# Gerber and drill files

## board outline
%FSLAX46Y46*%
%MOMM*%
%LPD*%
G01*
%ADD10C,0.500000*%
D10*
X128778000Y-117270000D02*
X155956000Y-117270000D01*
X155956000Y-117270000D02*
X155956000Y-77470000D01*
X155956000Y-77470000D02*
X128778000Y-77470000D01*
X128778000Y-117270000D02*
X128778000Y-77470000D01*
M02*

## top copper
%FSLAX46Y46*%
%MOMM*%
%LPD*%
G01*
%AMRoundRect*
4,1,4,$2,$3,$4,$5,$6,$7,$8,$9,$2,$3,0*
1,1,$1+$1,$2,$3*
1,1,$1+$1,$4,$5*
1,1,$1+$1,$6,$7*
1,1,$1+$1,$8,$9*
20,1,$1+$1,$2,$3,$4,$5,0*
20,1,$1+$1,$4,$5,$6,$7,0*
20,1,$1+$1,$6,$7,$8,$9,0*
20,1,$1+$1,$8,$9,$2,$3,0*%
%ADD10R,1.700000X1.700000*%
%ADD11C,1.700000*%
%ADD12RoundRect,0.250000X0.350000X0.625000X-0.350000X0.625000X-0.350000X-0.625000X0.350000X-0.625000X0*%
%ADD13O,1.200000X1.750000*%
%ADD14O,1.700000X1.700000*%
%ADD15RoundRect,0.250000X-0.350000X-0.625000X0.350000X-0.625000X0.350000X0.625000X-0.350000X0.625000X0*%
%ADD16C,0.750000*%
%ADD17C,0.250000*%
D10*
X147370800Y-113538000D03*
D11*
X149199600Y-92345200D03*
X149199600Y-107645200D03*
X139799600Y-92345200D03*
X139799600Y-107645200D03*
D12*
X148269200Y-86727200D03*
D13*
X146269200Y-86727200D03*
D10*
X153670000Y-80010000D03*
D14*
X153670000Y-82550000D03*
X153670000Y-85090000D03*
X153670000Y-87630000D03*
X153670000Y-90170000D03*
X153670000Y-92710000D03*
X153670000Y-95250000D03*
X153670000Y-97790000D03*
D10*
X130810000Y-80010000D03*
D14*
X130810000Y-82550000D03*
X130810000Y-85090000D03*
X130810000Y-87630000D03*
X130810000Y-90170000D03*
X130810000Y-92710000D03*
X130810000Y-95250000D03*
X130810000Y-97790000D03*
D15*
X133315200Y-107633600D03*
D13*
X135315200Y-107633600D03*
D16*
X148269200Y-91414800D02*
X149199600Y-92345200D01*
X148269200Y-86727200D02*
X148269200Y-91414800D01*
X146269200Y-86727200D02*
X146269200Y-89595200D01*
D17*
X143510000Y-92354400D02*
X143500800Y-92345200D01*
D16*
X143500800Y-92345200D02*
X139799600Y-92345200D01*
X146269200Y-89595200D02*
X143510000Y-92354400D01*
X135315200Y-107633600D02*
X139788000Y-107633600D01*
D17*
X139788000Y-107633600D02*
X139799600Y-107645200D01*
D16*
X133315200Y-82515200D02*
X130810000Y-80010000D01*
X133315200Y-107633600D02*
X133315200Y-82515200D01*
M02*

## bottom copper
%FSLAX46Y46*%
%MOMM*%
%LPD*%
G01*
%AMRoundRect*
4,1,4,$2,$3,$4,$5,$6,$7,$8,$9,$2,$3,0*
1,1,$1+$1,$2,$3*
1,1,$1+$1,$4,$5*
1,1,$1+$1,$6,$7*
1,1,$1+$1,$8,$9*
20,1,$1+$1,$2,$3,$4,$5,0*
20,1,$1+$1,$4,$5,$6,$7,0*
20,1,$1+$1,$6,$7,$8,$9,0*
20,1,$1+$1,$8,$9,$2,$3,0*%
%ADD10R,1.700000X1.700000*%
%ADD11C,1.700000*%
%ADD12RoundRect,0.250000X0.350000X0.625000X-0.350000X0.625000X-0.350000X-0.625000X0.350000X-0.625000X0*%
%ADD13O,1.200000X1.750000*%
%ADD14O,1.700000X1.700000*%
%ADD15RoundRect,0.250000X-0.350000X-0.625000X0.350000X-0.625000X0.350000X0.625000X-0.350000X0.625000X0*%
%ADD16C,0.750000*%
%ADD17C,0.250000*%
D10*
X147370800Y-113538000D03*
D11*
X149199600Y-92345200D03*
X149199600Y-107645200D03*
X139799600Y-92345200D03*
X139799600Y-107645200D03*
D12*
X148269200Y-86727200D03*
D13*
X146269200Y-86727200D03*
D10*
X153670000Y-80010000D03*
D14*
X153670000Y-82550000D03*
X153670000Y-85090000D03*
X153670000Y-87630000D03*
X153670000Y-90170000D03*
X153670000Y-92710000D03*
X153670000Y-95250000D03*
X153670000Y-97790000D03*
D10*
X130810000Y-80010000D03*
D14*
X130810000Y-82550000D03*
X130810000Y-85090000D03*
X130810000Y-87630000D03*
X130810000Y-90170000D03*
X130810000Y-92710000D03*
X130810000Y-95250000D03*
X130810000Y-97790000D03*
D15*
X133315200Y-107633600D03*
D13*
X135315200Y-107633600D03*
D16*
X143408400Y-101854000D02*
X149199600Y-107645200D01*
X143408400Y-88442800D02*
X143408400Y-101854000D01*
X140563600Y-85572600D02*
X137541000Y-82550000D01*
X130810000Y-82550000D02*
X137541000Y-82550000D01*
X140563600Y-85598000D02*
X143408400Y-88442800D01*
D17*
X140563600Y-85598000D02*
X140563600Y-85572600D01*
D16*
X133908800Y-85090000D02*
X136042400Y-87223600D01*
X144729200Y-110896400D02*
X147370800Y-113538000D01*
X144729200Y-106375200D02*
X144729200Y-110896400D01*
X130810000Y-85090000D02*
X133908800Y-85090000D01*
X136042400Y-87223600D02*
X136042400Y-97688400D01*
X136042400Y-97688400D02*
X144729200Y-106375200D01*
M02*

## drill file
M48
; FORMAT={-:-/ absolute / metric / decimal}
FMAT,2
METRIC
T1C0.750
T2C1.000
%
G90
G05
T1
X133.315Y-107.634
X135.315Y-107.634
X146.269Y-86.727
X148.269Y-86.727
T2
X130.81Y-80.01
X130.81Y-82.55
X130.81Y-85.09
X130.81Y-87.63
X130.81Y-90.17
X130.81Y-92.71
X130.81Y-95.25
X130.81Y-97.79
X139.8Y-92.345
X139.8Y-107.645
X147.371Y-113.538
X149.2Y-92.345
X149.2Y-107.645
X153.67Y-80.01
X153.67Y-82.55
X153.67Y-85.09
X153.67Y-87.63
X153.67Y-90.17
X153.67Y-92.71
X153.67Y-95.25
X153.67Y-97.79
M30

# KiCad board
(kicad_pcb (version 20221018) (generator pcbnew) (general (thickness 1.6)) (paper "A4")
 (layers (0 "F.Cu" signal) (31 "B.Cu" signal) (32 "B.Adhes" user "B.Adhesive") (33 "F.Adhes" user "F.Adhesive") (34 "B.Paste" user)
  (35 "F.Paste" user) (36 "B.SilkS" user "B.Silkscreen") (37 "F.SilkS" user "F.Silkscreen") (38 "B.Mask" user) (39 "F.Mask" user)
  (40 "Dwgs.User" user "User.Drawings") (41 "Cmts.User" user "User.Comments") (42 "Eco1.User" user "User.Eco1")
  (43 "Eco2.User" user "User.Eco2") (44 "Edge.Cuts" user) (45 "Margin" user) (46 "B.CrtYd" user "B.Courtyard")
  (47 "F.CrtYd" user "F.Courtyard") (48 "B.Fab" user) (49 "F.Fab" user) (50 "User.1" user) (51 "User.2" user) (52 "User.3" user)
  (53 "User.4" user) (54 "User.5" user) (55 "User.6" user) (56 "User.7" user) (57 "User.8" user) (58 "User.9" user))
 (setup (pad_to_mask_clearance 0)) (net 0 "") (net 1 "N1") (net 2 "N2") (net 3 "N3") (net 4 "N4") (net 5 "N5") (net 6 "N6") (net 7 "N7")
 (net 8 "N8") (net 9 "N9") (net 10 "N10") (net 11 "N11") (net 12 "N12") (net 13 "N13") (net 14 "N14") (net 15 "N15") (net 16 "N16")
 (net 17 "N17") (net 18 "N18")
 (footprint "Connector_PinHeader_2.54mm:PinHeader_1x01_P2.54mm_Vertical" (layer "F.Cu") (at 147.3708 113.538)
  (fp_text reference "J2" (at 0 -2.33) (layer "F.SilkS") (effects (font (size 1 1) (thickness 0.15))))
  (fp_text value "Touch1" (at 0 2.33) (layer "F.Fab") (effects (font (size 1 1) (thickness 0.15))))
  (pad "1" thru_hole rect (at 0 0) (size 1.7 1.7) (drill 1) (layers "*.Cu" "*.Mask") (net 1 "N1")))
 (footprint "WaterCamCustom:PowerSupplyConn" (layer "F.Cu") (at 144.4996 99.9952 -90)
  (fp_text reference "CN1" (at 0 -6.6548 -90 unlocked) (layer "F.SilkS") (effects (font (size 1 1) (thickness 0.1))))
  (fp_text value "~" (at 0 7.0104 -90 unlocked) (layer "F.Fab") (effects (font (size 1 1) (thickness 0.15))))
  (pad "1" thru_hole circle (at -7.65 -4.7 270) (size 1.7 1.7) (drill 1) (layers "*.Cu" "*.Mask") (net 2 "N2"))
  (pad "2" thru_hole circle (at 7.65 -4.7 270) (size 1.7 1.7) (drill 1) (layers "*.Cu" "*.Mask") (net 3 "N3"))
  (pad "3" thru_hole circle (at -7.65 4.7 270) (size 1.7 1.7) (drill 1) (layers "*.Cu" "*.Mask") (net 1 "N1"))
  (pad "4" thru_hole circle (at 7.65 4.7 270) (size 1.7 1.7) (drill 1) (layers "*.Cu" "*.Mask") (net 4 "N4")))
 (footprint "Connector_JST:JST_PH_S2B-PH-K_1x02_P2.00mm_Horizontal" (layer "F.Cu") (at 148.2692 86.7272 180)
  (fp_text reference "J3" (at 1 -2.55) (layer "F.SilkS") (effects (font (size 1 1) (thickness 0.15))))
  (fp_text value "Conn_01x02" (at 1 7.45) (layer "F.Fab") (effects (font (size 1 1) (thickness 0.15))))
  (pad "1" thru_hole roundrect (at 0 0 180) (size 1.2 1.75) (drill 0.75) (layers "*.Cu" "*.Mask") (roundrect_rratio 0.2083333333)
   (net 2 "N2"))
  (pad "2" thru_hole oval (at 2 0 180) (size 1.2 1.75) (drill 0.75) (layers "*.Cu" "*.Mask") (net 1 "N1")))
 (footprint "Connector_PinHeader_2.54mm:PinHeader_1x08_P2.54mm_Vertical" (layer "F.Cu") (at 153.67 80.01)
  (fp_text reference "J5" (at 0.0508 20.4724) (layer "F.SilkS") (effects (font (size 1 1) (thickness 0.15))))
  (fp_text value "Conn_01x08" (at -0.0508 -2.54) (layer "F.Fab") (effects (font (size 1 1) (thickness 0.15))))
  (pad "1" thru_hole rect (at 0 0) (size 1.7 1.7) (drill 1) (layers "*.Cu" "*.Mask") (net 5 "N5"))
  (pad "2" thru_hole oval (at 0 2.54) (size 1.7 1.7) (drill 1) (layers "*.Cu" "*.Mask") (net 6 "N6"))
  (pad "3" thru_hole oval (at 0 5.08) (size 1.7 1.7) (drill 1) (layers "*.Cu" "*.Mask") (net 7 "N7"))
  (pad "4" thru_hole oval (at 0 7.62) (size 1.7 1.7) (drill 1) (layers "*.Cu" "*.Mask") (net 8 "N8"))
  (pad "5" thru_hole oval (at 0 10.16) (size 1.7 1.7) (drill 1) (layers "*.Cu" "*.Mask") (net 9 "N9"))
  (pad "6" thru_hole oval (at 0 12.7) (size 1.7 1.7) (drill 1) (layers "*.Cu" "*.Mask") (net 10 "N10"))
  (pad "7" thru_hole oval (at 0 15.24) (size 1.7 1.7) (drill 1) (layers "*.Cu" "*.Mask") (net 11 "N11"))
  (pad "8" thru_hole oval (at 0 17.78) (size 1.7 1.7) (drill 1) (layers "*.Cu" "*.Mask") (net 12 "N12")))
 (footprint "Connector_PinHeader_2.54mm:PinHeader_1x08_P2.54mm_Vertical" (layer "F.Cu") (at 130.81 80.01)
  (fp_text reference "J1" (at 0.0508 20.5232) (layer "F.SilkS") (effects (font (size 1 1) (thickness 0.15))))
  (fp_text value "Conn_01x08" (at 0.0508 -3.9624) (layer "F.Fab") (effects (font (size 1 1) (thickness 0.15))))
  (pad "1" thru_hole rect (at 0 0) (size 1.7 1.7) (drill 1) (layers "*.Cu" "*.Mask") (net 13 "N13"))
  (pad "2" thru_hole oval (at 0 2.54) (size 1.7 1.7) (drill 1) (layers "*.Cu" "*.Mask") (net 3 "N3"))
  (pad "3" thru_hole oval (at 0 5.08) (size 1.7 1.7) (drill 1) (layers "*.Cu" "*.Mask") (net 1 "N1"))
  (pad "4" thru_hole oval (at 0 7.62) (size 1.7 1.7) (drill 1) (layers "*.Cu" "*.Mask") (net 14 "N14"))
  (pad "5" thru_hole oval (at 0 10.16) (size 1.7 1.7) (drill 1) (layers "*.Cu" "*.Mask") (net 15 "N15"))
  (pad "6" thru_hole oval (at 0 12.7) (size 1.7 1.7) (drill 1) (layers "*.Cu" "*.Mask") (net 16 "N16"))
  (pad "7" thru_hole oval (at 0 15.24) (size 1.7 1.7) (drill 1) (layers "*.Cu" "*.Mask") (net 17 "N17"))
  (pad "8" thru_hole oval (at 0 17.78) (size 1.7 1.7) (drill 1) (layers "*.Cu" "*.Mask") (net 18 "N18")))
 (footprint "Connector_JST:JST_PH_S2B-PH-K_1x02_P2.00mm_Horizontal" (layer "F.Cu") (at 133.3152 107.6336)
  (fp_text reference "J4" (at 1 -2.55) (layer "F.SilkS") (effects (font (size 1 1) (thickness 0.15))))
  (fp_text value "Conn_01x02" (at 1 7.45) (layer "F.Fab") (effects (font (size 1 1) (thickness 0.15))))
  (pad "1" thru_hole roundrect (at 0 0) (size 1.2 1.75) (drill 0.75) (layers "*.Cu" "*.Mask") (roundrect_rratio 0.2083333333) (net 13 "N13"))
  (pad "2" thru_hole oval (at 2 0) (size 1.2 1.75) (drill 0.75) (layers "*.Cu" "*.Mask") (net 4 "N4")))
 (gr_line (start 128.778 117.27) (end 155.956 117.27) (stroke (width 0.5) (type solid)) (layer "Edge.Cuts"))
 (gr_line (start 155.956 117.27) (end 155.956 77.47) (stroke (width 0.5) (type solid)) (layer "Edge.Cuts"))
 (gr_line (start 155.956 77.47) (end 128.778 77.47) (stroke (width 0.5) (type solid)) (layer "Edge.Cuts"))
 (gr_line (start 128.778 117.27) (end 128.778 77.47) (stroke (width 0.5) (type solid)) (layer "Edge.Cuts"))
 (segment (start 148.2692 91.4148) (end 149.1996 92.3452) (width 0.75) (layer "F.Cu") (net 2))
 (segment (start 148.2692 86.7272) (end 148.2692 91.4148) (width 0.75) (layer "F.Cu") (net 2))
 (segment (start 143.4084 101.854) (end 149.1996 107.6452) (width 0.75) (layer "B.Cu") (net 3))
 (segment (start 143.4084 88.4428) (end 143.4084 101.854) (width 0.75) (layer "B.Cu") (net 3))
 (segment (start 140.5636 85.5726) (end 137.541 82.55) (width 0.75) (layer "B.Cu") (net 3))
 (segment (start 130.81 82.55) (end 137.541 82.55) (width 0.75) (layer "B.Cu") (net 3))
 (segment (start 140.5636 85.598) (end 143.4084 88.4428) (width 0.75) (layer "B.Cu") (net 3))
 (segment (start 140.5636 85.598) (end 140.5636 85.5726) (width 0.25) (layer "B.Cu") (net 3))
 (segment (start 146.2692 86.7272) (end 146.2692 89.5952) (width 0.75) (layer "F.Cu") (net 1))
 (segment (start 143.51 92.3544) (end 143.5008 92.3452) (width 0.25) (layer "F.Cu") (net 1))
 (segment (start 143.5008 92.3452) (end 139.7996 92.3452) (width 0.75) (layer "F.Cu") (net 1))
 (segment (start 146.2692 89.5952) (end 143.51 92.3544) (width 0.75) (layer "F.Cu") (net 1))
 (segment (start 133.9088 85.09) (end 136.0424 87.2236) (width 0.75) (layer "B.Cu") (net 1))
 (segment (start 144.7292 110.8964) (end 147.3708 113.538) (width 0.75) (layer "B.Cu") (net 1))
 (segment (start 144.7292 106.3752) (end 144.7292 110.8964) (width 0.75) (layer "B.Cu") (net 1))
 (segment (start 130.81 85.09) (end 133.9088 85.09) (width 0.75) (layer "B.Cu") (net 1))
 (segment (start 136.0424 87.2236) (end 136.0424 97.6884) (width 0.75) (layer "B.Cu") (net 1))
 (segment (start 136.0424 97.6884) (end 144.7292 106.3752) (width 0.75) (layer "B.Cu") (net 1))
 (segment (start 135.3152 107.6336) (end 139.788 107.6336) (width 0.75) (layer "F.Cu") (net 4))
 (segment (start 139.788 107.6336) (end 139.7996 107.6452) (width 0.25) (layer "F.Cu") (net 4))
 (segment (start 133.3152 82.5152) (end 130.81 80.01) (width 0.75) (layer "F.Cu") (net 13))
 (segment (start 133.3152 107.6336) (end 133.3152 82.5152) (width 0.75) (layer "F.Cu") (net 13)))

